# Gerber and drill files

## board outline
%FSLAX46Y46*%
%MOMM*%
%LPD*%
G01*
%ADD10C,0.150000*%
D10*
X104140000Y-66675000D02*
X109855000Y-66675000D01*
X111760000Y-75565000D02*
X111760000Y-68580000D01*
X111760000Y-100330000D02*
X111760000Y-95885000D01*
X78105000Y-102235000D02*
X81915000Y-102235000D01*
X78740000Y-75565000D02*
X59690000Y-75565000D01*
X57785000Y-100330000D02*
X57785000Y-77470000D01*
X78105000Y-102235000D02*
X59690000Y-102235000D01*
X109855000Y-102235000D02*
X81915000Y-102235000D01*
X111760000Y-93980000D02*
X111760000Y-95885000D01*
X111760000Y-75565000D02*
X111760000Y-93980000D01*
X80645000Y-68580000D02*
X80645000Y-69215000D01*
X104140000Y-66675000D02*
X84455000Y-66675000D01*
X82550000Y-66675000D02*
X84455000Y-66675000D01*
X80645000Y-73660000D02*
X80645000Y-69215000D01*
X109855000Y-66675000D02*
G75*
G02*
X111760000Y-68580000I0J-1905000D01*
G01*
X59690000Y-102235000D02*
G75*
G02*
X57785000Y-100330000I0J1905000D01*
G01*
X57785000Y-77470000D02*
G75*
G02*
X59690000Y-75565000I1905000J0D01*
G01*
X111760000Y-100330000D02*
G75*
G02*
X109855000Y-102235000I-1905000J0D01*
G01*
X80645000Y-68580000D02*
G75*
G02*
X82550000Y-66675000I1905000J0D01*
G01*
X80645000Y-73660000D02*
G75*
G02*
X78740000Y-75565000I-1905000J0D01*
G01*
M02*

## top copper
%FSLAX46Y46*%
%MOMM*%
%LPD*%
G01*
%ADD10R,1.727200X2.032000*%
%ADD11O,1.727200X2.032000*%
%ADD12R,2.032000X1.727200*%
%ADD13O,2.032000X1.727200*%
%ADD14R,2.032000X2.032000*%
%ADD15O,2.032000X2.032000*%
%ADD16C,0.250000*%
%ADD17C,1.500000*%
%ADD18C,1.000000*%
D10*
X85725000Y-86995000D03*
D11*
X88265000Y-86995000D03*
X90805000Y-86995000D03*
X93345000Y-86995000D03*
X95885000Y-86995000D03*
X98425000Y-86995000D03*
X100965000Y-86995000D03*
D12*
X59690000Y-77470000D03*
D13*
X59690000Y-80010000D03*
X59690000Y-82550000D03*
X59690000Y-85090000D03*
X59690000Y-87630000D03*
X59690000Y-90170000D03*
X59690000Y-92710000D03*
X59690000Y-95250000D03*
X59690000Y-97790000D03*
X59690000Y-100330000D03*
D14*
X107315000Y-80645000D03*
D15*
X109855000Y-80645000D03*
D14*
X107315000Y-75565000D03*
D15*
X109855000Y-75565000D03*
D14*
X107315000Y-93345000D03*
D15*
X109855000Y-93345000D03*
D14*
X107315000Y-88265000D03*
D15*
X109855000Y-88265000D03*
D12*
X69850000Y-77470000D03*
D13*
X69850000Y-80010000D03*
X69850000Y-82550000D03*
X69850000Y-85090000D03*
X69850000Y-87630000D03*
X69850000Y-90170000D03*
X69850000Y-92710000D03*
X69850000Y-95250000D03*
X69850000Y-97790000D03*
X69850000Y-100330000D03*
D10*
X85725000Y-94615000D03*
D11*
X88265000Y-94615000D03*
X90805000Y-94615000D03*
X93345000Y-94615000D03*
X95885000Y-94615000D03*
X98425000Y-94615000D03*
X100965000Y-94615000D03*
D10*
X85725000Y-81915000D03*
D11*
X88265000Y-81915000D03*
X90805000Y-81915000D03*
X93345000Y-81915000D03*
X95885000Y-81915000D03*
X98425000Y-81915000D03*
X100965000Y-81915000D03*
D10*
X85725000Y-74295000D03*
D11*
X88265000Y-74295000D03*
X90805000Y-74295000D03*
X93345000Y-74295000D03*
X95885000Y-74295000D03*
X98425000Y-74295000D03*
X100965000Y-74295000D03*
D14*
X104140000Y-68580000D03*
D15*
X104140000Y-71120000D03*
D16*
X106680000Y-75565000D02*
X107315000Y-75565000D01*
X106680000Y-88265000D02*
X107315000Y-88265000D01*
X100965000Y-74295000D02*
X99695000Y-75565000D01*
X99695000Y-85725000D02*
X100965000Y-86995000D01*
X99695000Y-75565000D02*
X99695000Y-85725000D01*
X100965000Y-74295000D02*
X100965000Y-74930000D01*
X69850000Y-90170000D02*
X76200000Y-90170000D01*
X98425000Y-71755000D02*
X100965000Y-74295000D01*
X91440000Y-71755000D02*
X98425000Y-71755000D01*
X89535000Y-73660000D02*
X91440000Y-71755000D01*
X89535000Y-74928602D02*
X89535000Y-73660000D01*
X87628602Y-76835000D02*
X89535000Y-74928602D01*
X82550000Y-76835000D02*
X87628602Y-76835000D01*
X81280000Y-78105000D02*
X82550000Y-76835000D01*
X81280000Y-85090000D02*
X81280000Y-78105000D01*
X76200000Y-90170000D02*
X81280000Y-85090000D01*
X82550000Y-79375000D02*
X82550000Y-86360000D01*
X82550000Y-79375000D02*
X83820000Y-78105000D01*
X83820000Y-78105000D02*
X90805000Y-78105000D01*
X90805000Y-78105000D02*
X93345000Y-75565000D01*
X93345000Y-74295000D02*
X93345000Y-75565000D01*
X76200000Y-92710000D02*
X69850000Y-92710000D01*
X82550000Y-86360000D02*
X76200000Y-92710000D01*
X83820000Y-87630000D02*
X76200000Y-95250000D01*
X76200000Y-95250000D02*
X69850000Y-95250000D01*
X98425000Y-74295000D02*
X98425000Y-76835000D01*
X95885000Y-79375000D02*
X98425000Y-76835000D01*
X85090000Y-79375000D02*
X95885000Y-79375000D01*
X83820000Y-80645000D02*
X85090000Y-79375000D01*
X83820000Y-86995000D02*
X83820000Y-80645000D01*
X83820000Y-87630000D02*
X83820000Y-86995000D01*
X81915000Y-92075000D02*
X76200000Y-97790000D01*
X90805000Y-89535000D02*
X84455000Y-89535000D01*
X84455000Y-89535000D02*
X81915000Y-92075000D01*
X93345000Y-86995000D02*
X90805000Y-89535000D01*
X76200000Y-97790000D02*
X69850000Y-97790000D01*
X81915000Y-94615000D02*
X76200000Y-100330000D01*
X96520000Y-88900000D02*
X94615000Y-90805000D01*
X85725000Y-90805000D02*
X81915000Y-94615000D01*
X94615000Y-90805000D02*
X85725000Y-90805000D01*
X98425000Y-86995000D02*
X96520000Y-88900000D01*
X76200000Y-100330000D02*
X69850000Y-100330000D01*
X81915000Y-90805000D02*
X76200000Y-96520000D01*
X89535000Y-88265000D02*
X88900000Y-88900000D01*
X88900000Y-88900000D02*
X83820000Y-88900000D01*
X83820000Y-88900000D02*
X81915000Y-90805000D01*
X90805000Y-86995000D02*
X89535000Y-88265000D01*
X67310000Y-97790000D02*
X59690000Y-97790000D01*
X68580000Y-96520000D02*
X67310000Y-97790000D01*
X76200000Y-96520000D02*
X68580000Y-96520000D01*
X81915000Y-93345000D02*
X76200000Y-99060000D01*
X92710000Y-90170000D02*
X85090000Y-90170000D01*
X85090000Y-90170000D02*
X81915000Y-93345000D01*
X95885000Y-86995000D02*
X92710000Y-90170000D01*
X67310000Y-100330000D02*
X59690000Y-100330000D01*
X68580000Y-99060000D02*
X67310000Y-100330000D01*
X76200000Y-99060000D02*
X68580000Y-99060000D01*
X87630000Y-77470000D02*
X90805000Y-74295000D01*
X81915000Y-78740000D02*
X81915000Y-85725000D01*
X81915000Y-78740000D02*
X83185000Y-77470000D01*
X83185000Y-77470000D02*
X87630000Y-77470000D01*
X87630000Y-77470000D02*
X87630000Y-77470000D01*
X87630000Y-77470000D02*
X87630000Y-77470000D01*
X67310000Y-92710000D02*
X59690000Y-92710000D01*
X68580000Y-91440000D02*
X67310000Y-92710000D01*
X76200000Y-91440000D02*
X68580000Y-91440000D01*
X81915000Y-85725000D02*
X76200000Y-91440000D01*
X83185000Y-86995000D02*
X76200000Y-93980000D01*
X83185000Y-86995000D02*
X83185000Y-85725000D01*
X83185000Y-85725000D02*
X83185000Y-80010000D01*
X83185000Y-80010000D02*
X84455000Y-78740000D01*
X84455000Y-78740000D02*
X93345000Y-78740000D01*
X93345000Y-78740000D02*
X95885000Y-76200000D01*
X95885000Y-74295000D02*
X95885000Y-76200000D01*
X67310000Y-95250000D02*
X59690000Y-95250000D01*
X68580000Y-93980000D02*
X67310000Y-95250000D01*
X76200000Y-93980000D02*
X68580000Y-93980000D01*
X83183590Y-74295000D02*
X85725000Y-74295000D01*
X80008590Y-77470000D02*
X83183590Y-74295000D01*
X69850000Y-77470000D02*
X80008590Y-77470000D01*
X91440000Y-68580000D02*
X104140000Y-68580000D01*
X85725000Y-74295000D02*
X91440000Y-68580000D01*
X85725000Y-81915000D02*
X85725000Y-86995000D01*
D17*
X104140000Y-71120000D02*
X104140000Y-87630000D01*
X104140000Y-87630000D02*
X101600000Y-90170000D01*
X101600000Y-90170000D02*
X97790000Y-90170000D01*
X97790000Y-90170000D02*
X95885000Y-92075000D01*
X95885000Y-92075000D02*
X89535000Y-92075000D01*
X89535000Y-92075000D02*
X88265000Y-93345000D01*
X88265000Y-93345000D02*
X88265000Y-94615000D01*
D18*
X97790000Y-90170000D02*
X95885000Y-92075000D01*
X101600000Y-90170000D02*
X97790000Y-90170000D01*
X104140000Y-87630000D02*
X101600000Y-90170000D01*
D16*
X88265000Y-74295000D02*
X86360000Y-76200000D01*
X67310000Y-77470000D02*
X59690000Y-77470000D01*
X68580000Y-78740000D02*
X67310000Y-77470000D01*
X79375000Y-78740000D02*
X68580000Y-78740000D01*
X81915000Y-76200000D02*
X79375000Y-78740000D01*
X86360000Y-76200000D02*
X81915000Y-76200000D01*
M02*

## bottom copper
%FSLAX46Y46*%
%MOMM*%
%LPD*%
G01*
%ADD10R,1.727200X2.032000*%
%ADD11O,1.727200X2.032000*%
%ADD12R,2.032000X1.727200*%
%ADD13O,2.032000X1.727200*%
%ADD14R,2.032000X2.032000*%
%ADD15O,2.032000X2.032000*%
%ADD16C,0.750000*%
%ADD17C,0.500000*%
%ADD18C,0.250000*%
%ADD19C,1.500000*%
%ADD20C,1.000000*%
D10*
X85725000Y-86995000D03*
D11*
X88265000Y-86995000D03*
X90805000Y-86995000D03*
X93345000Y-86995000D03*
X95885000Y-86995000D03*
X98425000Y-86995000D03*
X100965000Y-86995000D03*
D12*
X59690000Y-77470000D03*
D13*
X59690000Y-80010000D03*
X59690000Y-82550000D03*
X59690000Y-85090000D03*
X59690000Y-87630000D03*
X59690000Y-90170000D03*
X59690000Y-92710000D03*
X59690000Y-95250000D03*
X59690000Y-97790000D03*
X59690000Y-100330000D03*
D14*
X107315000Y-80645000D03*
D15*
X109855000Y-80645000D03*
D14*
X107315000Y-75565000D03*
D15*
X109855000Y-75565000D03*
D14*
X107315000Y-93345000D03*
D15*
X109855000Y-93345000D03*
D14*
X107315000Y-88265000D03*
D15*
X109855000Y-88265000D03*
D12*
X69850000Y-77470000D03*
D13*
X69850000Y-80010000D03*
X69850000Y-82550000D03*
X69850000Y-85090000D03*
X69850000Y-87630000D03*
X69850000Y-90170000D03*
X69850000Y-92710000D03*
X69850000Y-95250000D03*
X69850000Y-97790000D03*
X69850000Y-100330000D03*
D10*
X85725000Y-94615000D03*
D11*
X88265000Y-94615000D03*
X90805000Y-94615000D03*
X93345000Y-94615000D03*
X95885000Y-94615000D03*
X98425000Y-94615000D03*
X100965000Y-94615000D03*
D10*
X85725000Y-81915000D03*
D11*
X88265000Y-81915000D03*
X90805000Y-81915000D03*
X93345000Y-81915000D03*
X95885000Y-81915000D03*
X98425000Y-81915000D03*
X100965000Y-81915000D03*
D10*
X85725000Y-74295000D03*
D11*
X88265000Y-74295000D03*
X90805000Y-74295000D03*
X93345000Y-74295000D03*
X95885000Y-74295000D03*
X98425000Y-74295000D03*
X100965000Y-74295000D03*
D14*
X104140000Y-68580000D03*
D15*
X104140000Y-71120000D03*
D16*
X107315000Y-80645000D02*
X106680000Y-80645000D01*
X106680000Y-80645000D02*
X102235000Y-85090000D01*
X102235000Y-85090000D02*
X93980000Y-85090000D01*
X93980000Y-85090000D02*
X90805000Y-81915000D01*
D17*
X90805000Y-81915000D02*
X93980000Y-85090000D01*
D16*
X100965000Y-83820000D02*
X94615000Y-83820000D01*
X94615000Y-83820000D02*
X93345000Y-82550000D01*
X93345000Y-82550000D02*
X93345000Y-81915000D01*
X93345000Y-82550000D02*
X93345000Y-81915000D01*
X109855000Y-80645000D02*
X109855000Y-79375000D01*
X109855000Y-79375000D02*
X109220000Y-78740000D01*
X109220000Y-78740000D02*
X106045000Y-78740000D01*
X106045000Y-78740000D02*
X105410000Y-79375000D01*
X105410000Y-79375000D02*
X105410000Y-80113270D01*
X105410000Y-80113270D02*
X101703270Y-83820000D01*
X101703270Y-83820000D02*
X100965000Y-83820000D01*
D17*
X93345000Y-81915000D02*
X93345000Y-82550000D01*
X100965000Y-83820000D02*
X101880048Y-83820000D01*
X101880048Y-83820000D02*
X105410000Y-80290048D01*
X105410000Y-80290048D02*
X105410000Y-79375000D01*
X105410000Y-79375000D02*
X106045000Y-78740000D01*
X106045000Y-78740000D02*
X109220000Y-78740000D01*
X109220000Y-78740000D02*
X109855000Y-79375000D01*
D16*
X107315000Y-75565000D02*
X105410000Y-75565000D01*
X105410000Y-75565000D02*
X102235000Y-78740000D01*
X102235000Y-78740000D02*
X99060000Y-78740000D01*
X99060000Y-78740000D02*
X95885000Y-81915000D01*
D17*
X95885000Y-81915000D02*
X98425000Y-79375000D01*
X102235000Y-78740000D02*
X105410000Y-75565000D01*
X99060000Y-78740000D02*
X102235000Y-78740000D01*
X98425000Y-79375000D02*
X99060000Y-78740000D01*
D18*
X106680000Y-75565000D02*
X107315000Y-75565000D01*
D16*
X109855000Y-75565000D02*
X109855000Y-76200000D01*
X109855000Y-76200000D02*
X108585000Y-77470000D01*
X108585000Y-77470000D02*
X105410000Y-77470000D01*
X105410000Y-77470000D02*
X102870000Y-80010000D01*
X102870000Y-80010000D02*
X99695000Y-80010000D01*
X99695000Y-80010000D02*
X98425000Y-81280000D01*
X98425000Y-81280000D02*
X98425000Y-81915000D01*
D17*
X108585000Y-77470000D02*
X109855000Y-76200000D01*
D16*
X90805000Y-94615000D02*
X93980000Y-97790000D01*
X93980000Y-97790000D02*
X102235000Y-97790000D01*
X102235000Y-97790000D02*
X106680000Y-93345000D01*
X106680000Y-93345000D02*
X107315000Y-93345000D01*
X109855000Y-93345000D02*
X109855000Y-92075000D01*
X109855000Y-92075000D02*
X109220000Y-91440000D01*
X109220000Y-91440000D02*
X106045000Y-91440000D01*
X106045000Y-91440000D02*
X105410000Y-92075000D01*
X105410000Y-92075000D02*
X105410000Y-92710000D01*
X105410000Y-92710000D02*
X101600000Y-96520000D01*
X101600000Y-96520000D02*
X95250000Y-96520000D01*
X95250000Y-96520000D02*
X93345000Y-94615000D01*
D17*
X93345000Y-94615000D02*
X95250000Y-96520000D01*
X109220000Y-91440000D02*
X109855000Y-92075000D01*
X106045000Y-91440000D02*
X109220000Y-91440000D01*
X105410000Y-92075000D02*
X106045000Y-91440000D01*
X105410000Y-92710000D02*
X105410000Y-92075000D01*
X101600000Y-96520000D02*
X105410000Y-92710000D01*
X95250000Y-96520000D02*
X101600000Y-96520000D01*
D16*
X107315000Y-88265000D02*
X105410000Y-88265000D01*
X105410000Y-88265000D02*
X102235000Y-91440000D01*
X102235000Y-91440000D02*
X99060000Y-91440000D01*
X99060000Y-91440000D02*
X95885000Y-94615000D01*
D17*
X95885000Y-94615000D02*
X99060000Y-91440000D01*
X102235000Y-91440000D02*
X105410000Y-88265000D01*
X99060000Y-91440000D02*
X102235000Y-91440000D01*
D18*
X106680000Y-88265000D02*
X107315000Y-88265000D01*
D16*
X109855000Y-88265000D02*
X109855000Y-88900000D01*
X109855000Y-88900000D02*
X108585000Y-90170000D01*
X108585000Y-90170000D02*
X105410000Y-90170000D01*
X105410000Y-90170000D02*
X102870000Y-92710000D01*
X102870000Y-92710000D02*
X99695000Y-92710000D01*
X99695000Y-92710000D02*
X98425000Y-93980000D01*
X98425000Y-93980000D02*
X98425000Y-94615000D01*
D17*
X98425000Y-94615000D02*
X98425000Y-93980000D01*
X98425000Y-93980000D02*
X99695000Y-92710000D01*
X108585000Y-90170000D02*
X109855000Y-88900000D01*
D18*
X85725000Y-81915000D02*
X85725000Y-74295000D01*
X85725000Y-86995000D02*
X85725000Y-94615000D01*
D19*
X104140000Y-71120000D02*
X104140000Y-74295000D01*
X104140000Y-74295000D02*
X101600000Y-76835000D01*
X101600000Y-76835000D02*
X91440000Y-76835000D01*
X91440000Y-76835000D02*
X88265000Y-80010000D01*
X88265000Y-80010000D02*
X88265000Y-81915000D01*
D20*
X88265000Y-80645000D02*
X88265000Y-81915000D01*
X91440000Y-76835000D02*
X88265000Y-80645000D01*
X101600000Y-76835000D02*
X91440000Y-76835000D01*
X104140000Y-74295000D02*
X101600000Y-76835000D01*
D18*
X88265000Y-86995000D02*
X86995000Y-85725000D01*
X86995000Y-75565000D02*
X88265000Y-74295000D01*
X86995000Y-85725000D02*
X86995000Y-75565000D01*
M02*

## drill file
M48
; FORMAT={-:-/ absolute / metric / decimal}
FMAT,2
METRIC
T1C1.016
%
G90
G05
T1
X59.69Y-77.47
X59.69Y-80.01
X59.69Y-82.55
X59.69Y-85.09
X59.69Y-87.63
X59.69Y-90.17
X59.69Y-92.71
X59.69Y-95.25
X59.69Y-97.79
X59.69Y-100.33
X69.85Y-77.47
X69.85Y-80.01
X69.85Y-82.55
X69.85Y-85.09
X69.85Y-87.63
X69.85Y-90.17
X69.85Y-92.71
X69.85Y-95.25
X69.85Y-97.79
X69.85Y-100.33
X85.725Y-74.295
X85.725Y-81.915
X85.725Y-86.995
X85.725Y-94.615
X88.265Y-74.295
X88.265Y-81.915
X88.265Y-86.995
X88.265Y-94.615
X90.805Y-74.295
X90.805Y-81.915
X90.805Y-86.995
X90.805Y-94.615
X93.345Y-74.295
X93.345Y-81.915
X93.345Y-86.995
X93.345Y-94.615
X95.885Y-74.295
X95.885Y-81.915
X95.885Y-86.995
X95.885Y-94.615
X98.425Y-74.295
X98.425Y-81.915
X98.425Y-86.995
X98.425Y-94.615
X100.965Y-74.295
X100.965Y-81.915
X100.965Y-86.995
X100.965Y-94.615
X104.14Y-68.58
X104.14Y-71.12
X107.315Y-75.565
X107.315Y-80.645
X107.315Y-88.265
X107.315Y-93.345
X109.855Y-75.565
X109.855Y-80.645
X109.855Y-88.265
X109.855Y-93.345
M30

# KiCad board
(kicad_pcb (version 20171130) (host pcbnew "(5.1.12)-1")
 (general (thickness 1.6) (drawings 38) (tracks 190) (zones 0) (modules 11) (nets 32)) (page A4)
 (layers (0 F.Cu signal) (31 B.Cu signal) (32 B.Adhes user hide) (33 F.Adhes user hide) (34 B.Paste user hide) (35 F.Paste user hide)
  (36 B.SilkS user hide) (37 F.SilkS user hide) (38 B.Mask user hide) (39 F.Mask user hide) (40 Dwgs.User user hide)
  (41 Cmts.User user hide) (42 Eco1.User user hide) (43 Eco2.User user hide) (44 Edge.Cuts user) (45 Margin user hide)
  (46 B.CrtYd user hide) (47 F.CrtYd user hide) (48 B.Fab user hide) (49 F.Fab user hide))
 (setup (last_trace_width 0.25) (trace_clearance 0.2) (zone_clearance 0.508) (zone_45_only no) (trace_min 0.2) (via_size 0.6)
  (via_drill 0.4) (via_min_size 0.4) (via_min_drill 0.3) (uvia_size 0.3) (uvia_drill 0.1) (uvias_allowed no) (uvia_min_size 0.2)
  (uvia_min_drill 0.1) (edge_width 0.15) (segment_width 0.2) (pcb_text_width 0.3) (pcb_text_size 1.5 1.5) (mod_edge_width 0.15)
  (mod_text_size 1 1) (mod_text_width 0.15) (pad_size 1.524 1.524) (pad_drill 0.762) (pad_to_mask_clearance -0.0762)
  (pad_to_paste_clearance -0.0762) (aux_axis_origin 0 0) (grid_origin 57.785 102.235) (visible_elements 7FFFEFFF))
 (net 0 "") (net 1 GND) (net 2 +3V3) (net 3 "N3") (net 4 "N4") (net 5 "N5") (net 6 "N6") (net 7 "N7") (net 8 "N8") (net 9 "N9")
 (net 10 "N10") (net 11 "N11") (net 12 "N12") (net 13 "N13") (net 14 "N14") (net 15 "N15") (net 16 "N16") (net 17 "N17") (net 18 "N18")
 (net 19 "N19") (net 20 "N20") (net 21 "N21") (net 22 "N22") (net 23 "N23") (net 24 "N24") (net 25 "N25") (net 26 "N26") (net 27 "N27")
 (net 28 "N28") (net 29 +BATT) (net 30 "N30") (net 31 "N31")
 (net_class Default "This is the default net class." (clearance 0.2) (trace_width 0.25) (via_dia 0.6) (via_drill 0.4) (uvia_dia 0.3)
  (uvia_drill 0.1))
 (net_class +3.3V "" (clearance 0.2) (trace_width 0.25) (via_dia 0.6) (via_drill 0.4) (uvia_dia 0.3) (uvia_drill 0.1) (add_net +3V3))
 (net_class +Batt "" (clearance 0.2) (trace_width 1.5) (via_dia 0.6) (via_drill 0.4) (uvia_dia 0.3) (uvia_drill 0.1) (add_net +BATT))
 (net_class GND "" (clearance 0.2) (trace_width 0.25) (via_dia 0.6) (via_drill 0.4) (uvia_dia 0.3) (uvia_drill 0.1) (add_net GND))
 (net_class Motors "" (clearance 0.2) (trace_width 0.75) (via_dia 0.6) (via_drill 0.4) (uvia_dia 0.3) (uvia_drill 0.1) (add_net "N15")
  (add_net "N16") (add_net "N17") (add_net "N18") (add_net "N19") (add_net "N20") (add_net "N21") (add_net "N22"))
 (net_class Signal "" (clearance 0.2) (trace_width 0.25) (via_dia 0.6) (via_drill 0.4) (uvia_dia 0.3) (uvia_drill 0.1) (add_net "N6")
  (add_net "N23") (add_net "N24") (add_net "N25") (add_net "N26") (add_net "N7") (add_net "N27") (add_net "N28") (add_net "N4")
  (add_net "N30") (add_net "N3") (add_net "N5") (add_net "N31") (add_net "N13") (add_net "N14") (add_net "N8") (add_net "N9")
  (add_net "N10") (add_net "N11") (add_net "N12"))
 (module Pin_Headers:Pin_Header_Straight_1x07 (layer F.Cu) (at 85.725 86.995 90)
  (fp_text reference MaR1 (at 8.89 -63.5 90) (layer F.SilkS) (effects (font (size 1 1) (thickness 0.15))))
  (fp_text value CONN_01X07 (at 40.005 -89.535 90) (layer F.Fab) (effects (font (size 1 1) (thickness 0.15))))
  (pad 1 thru_hole rect (at 0 0 90) (size 2.032 1.7272) (drill 1.016) (layers *.Cu *.Mask F.SilkS) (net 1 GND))
  (pad 2 thru_hole oval (at 0 2.54 90) (size 2.032 1.7272) (drill 1.016) (layers *.Cu *.Mask F.SilkS) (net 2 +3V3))
  (pad 3 thru_hole oval (at 0 5.08 90) (size 2.032 1.7272) (drill 1.016) (layers *.Cu *.Mask F.SilkS) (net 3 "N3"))
  (pad 4 thru_hole oval (at 0 7.62 90) (size 2.032 1.7272) (drill 1.016) (layers *.Cu *.Mask F.SilkS) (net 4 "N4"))
  (pad 5 thru_hole oval (at 0 10.16 90) (size 2.032 1.7272) (drill 1.016) (layers *.Cu *.Mask F.SilkS) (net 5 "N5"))
  (pad 6 thru_hole oval (at 0 12.7 90) (size 2.032 1.7272) (drill 1.016) (layers *.Cu *.Mask F.SilkS) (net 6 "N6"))
  (pad 7 thru_hole oval (at 0 15.24 90) (size 2.032 1.7272) (drill 1.016) (layers *.Cu *.Mask F.SilkS) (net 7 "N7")))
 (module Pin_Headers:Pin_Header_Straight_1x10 (layer F.Cu) (at 59.69 77.47)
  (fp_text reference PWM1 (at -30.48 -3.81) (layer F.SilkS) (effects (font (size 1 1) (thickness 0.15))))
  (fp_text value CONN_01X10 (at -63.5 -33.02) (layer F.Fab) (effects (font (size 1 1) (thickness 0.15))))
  (pad 1 thru_hole rect (at 0 0) (size 2.032 1.7272) (drill 1.016) (layers *.Cu *.Mask F.SilkS) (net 2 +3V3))
  (pad 2 thru_hole oval (at 0 2.54) (size 2.032 1.7272) (drill 1.016) (layers *.Cu *.Mask F.SilkS) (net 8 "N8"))
  (pad 3 thru_hole oval (at 0 5.08) (size 2.032 1.7272) (drill 1.016) (layers *.Cu *.Mask F.SilkS) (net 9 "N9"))
  (pad 4 thru_hole oval (at 0 7.62) (size 2.032 1.7272) (drill 1.016) (layers *.Cu *.Mask F.SilkS) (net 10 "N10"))
  (pad 5 thru_hole oval (at 0 10.16) (size 2.032 1.7272) (drill 1.016) (layers *.Cu *.Mask F.SilkS) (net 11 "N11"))
  (pad 6 thru_hole oval (at 0 12.7) (size 2.032 1.7272) (drill 1.016) (layers *.Cu *.Mask F.SilkS) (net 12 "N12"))
  (pad 7 thru_hole oval (at 0 15.24) (size 2.032 1.7272) (drill 1.016) (layers *.Cu *.Mask F.SilkS) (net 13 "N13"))
  (pad 8 thru_hole oval (at 0 17.78) (size 2.032 1.7272) (drill 1.016) (layers *.Cu *.Mask F.SilkS) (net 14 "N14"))
  (pad 9 thru_hole oval (at 0 20.32) (size 2.032 1.7272) (drill 1.016) (layers *.Cu *.Mask F.SilkS) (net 3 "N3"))
  (pad 10 thru_hole oval (at 0 22.86) (size 2.032 1.7272) (drill 1.016) (layers *.Cu *.Mask F.SilkS) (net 5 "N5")))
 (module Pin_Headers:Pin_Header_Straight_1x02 (layer F.Cu) (at 107.315 80.645 90)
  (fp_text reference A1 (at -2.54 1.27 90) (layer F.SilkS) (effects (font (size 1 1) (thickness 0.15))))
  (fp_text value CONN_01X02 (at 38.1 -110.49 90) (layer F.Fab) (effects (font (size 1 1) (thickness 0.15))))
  (pad 1 thru_hole rect (at 0 0 90) (size 2.032 2.032) (drill 1.016) (layers *.Cu *.Mask F.SilkS) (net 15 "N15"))
  (pad 2 thru_hole oval (at 0 2.54 90) (size 2.032 2.032) (drill 1.016) (layers *.Cu *.Mask F.SilkS) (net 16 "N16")))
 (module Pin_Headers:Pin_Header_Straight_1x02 (layer F.Cu) (at 107.315 75.565 90)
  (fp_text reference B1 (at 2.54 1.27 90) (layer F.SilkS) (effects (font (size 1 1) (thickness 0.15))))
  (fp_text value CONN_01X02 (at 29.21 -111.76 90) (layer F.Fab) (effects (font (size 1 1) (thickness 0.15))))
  (pad 1 thru_hole rect (at 0 0 90) (size 2.032 2.032) (drill 1.016) (layers *.Cu *.Mask F.SilkS) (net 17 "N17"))
  (pad 2 thru_hole oval (at 0 2.54 90) (size 2.032 2.032) (drill 1.016) (layers *.Cu *.Mask F.SilkS) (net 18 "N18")))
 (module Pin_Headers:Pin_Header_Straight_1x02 (layer F.Cu) (at 107.315 93.345 90)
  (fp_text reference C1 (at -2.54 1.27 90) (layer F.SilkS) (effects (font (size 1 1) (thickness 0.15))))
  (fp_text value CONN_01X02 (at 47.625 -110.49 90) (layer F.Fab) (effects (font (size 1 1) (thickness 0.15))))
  (pad 1 thru_hole rect (at 0 0 90) (size 2.032 2.032) (drill 1.016) (layers *.Cu *.Mask F.SilkS) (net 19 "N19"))
  (pad 2 thru_hole oval (at 0 2.54 90) (size 2.032 2.032) (drill 1.016) (layers *.Cu *.Mask F.SilkS) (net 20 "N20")))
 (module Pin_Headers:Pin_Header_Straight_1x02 (layer F.Cu) (at 107.315 88.265 90)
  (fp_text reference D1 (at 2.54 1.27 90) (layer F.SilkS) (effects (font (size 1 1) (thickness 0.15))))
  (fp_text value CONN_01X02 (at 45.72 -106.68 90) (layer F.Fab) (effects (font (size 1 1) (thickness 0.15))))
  (pad 1 thru_hole rect (at 0 0 90) (size 2.032 2.032) (drill 1.016) (layers *.Cu *.Mask F.SilkS) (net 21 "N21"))
  (pad 2 thru_hole oval (at 0 2.54 90) (size 2.032 2.032) (drill 1.016) (layers *.Cu *.Mask F.SilkS) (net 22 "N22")))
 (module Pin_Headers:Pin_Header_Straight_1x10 (layer F.Cu) (at 69.85 77.47)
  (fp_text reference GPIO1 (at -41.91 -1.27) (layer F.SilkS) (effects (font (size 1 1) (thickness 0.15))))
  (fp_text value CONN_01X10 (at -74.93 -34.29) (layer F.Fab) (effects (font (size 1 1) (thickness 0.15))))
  (pad 1 thru_hole rect (at 0 0) (size 2.032 1.7272) (drill 1.016) (layers *.Cu *.Mask F.SilkS) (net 1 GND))
  (pad 2 thru_hole oval (at 0 2.54) (size 2.032 1.7272) (drill 1.016) (layers *.Cu *.Mask F.SilkS) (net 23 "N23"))
  (pad 3 thru_hole oval (at 0 5.08) (size 2.032 1.7272) (drill 1.016) (layers *.Cu *.Mask F.SilkS) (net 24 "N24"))
  (pad 4 thru_hole oval (at 0 7.62) (size 2.032 1.7272) (drill 1.016) (layers *.Cu *.Mask F.SilkS) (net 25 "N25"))
  (pad 5 thru_hole oval (at 0 10.16) (size 2.032 1.7272) (drill 1.016) (layers *.Cu *.Mask F.SilkS) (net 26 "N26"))
  (pad 6 thru_hole oval (at 0 12.7) (size 2.032 1.7272) (drill 1.016) (layers *.Cu *.Mask F.SilkS) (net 7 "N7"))
  (pad 7 thru_hole oval (at 0 15.24) (size 2.032 1.7272) (drill 1.016) (layers *.Cu *.Mask F.SilkS) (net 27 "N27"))
  (pad 8 thru_hole oval (at 0 17.78) (size 2.032 1.7272) (drill 1.016) (layers *.Cu *.Mask F.SilkS) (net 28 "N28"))
  (pad 9 thru_hole oval (at 0 20.32) (size 2.032 1.7272) (drill 1.016) (layers *.Cu *.Mask F.SilkS) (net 4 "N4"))
  (pad 10 thru_hole oval (at 0 22.86) (size 2.032 1.7272) (drill 1.016) (layers *.Cu *.Mask F.SilkS) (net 6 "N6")))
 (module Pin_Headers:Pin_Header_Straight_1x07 (layer F.Cu) (at 85.725 94.615 90)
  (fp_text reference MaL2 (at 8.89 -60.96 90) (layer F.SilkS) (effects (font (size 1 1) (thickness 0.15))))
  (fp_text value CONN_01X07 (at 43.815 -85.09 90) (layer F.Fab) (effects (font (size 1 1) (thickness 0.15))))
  (pad 1 thru_hole rect (at 0 0 90) (size 2.032 1.7272) (drill 1.016) (layers *.Cu *.Mask F.SilkS) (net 1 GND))
  (pad 2 thru_hole oval (at 0 2.54 90) (size 2.032 1.7272) (drill 1.016) (layers *.Cu *.Mask F.SilkS) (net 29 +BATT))
  (pad 3 thru_hole oval (at 0 5.08 90) (size 2.032 1.7272) (drill 1.016) (layers *.Cu *.Mask F.SilkS) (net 19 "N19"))
  (pad 4 thru_hole oval (at 0 7.62 90) (size 2.032 1.7272) (drill 1.016) (layers *.Cu *.Mask F.SilkS) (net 20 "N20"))
  (pad 5 thru_hole oval (at 0 10.16 90) (size 2.032 1.7272) (drill 1.016) (layers *.Cu *.Mask F.SilkS) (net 21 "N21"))
  (pad 6 thru_hole oval (at 0 12.7 90) (size 2.032 1.7272) (drill 1.016) (layers *.Cu *.Mask F.SilkS) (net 22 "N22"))
  (pad 7 thru_hole oval (at 0 15.24 90) (size 2.032 1.7272) (drill 1.016) (layers *.Cu *.Mask F.SilkS) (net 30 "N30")))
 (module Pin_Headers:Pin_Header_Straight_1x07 (layer F.Cu) (at 85.725 81.915 90)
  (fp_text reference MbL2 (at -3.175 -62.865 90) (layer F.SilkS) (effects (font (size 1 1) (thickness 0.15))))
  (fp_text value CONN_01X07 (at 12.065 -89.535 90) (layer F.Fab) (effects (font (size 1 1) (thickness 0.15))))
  (pad 1 thru_hole rect (at 0 0 90) (size 2.032 1.7272) (drill 1.016) (layers *.Cu *.Mask F.SilkS) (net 1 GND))
  (pad 2 thru_hole oval (at 0 2.54 90) (size 2.032 1.7272) (drill 1.016) (layers *.Cu *.Mask F.SilkS) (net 29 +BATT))
  (pad 3 thru_hole oval (at 0 5.08 90) (size 2.032 1.7272) (drill 1.016) (layers *.Cu *.Mask F.SilkS) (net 15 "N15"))
  (pad 4 thru_hole oval (at 0 7.62 90) (size 2.032 1.7272) (drill 1.016) (layers *.Cu *.Mask F.SilkS) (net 16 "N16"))
  (pad 5 thru_hole oval (at 0 10.16 90) (size 2.032 1.7272) (drill 1.016) (layers *.Cu *.Mask F.SilkS) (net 17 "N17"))
  (pad 6 thru_hole oval (at 0 12.7 90) (size 2.032 1.7272) (drill 1.016) (layers *.Cu *.Mask F.SilkS) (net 18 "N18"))
  (pad 7 thru_hole oval (at 0 15.24 90) (size 2.032 1.7272) (drill 1.016) (layers *.Cu *.Mask F.SilkS) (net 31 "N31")))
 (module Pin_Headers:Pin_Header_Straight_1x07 (layer F.Cu) (at 85.725 74.295 90)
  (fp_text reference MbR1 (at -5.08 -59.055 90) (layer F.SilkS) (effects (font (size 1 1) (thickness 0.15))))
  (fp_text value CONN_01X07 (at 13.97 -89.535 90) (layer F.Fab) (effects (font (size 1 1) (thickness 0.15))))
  (pad 1 thru_hole rect (at 0 0 90) (size 2.032 1.7272) (drill 1.016) (layers *.Cu *.Mask F.SilkS) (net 1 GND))
  (pad 2 thru_hole oval (at 0 2.54 90) (size 2.032 1.7272) (drill 1.016) (layers *.Cu *.Mask F.SilkS) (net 2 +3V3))
  (pad 3 thru_hole oval (at 0 5.08 90) (size 2.032 1.7272) (drill 1.016) (layers *.Cu *.Mask F.SilkS) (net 13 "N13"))
  (pad 4 thru_hole oval (at 0 7.62 90) (size 2.032 1.7272) (drill 1.016) (layers *.Cu *.Mask F.SilkS) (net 27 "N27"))
  (pad 5 thru_hole oval (at 0 10.16 90) (size 2.032 1.7272) (drill 1.016) (layers *.Cu *.Mask F.SilkS) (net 14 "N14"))
  (pad 6 thru_hole oval (at 0 12.7 90) (size 2.032 1.7272) (drill 1.016) (layers *.Cu *.Mask F.SilkS) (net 28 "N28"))
  (pad 7 thru_hole oval (at 0 15.24 90) (size 2.032 1.7272) (drill 1.016) (layers *.Cu *.Mask F.SilkS) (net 7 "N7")))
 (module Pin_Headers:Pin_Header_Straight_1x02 (layer F.Cu) (at 104.14 68.58)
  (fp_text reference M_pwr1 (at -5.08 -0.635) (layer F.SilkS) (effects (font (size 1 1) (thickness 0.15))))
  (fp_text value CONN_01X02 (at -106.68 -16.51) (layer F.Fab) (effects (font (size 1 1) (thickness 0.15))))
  (pad 1 thru_hole rect (at 0 0) (size 2.032 2.032) (drill 1.016) (layers *.Cu *.Mask F.SilkS) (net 1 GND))
  (pad 2 thru_hole oval (at 0 2.54) (size 2.032 2.032) (drill 1.016) (layers *.Cu *.Mask F.SilkS) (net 29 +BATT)))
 (gr_line (start 104.14 66.675) (end 109.855 66.675) (angle 90) (layer Edge.Cuts) (width 0.15))
 (gr_line (start 111.76 75.565) (end 111.76 68.58) (angle 90) (layer Edge.Cuts) (width 0.15))
 (gr_line (start 111.76 100.33) (end 111.76 95.885) (angle 90) (layer Edge.Cuts) (width 0.15))
 (gr_line (start 78.105 102.235) (end 81.915 102.235) (angle 90) (layer Edge.Cuts) (width 0.15))
 (gr_line (start 78.74 75.565) (end 59.69 75.565) (angle 90) (layer Edge.Cuts) (width 0.15))
 (gr_line (start 57.785 100.33) (end 57.785 77.47) (angle 90) (layer Edge.Cuts) (width 0.15))
 (gr_line (start 78.105 102.235) (end 59.69 102.235) (angle 90) (layer Edge.Cuts) (width 0.15))
 (gr_line (start 109.855 102.235) (end 81.915 102.235) (angle 90) (layer Edge.Cuts) (width 0.15))
 (gr_line (start 111.76 93.98) (end 111.76 95.885) (angle 90) (layer Edge.Cuts) (width 0.15))
 (gr_line (start 111.76 75.565) (end 111.76 93.98) (angle 90) (layer Edge.Cuts) (width 0.15))
 (gr_line (start 80.645 68.58) (end 80.645 69.215) (angle 90) (layer Edge.Cuts) (width 0.15))
 (gr_line (start 104.14 66.675) (end 84.455 66.675) (angle 90) (layer Edge.Cuts) (width 0.15))
 (gr_line (start 82.55 66.675) (end 84.455 66.675) (angle 90) (layer Edge.Cuts) (width 0.15))
 (gr_line (start 80.645 73.66) (end 80.645 69.215) (angle 90) (layer Edge.Cuts) (width 0.15))
 (gr_arc (start 109.855 68.58) (end 109.855 66.675) (angle 90) (layer Edge.Cuts) (width 0.15))
 (gr_arc (start 59.69 100.33) (end 59.69 102.235) (angle 90) (layer Edge.Cuts) (width 0.15))
 (gr_arc (start 59.69 77.47) (end 57.785 77.47) (angle 90) (layer Edge.Cuts) (width 0.15))
 (gr_arc (start 109.855 100.33) (end 111.76 100.33) (angle 90) (layer Edge.Cuts) (width 0.15))
 (gr_arc (start 82.55 68.58) (end 80.645 68.58) (angle 90) (layer Edge.Cuts) (width 0.15))
 (gr_arc (start 78.74 73.66) (end 80.645 73.66) (angle 90) (layer Edge.Cuts) (width 0.15))
 (segment (start 107.315 80.645) (end 106.68 80.645) (width 0.75) (layer B.Cu) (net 15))
 (segment (start 106.68 80.645) (end 102.235 85.09) (width 0.75) (layer B.Cu) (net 15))
 (segment (start 102.235 85.09) (end 93.98 85.09) (width 0.75) (layer B.Cu) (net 15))
 (segment (start 93.98 85.09) (end 90.805 81.915) (width 0.75) (layer B.Cu) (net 15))
 (segment (start 90.805 81.915) (end 93.98 85.09) (width 0.5) (layer B.Cu) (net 15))
 (segment (start 100.965 83.82) (end 94.615 83.82) (width 0.75) (layer B.Cu) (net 16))
 (segment (start 94.615 83.82) (end 93.345 82.55) (width 0.75) (layer B.Cu) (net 16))
 (segment (start 93.345 82.55) (end 93.345 81.915) (width 0.75) (layer B.Cu) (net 16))
 (segment (start 93.345 82.55) (end 93.345 81.915) (width 0.75) (layer B.Cu) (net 16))
 (segment (start 109.855 80.645) (end 109.855 79.375) (width 0.75) (layer B.Cu) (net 16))
 (segment (start 109.855 79.375) (end 109.22 78.74) (width 0.75) (layer B.Cu) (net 16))
 (segment (start 109.22 78.74) (end 106.045 78.74) (width 0.75) (layer B.Cu) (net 16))
 (segment (start 106.045 78.74) (end 105.41 79.375) (width 0.75) (layer B.Cu) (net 16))
 (segment (start 105.41 79.375) (end 105.41 80.11327) (width 0.75) (layer B.Cu) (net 16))
 (segment (start 105.41 80.11327) (end 101.70327 83.82) (width 0.75) (layer B.Cu) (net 16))
 (segment (start 101.70327 83.82) (end 100.965 83.82) (width 0.75) (layer B.Cu) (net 16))
 (segment (start 93.345 81.915) (end 93.345 82.55) (width 0.5) (layer B.Cu) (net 16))
 (segment (start 100.965 83.82) (end 101.880048 83.82) (width 0.5) (layer B.Cu) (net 16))
 (segment (start 101.880048 83.82) (end 105.41 80.290048) (width 0.5) (layer B.Cu) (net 16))
 (segment (start 105.41 80.290048) (end 105.41 79.375) (width 0.5) (layer B.Cu) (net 16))
 (segment (start 105.41 79.375) (end 106.045 78.74) (width 0.5) (layer B.Cu) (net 16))
 (segment (start 106.045 78.74) (end 109.22 78.74) (width 0.5) (layer B.Cu) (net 16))
 (segment (start 109.22 78.74) (end 109.855 79.375) (width 0.5) (layer B.Cu) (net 16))
 (segment (start 107.315 75.565) (end 105.41 75.565) (width 0.75) (layer B.Cu) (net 17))
 (segment (start 105.41 75.565) (end 102.235 78.74) (width 0.75) (layer B.Cu) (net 17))
 (segment (start 102.235 78.74) (end 99.06 78.74) (width 0.75) (layer B.Cu) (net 17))
 (segment (start 99.06 78.74) (end 95.885 81.915) (width 0.75) (layer B.Cu) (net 17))
 (segment (start 95.885 81.915) (end 98.425 79.375) (width 0.5) (layer B.Cu) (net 17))
 (segment (start 102.235 78.74) (end 105.41 75.565) (width 0.5) (layer B.Cu) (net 17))
 (segment (start 99.06 78.74) (end 102.235 78.74) (width 0.5) (layer B.Cu) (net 17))
 (segment (start 98.425 79.375) (end 99.06 78.74) (width 0.5) (layer B.Cu) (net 17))
 (segment (start 106.68 75.565) (end 107.315 75.565) (width 0.25) (layer B.Cu) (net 17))
 (segment (start 106.68 75.565) (end 107.315 75.565) (width 0.25) (layer F.Cu) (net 17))
 (segment (start 109.855 75.565) (end 109.855 76.2) (width 0.75) (layer B.Cu) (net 18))
 (segment (start 109.855 76.2) (end 108.585 77.47) (width 0.75) (layer B.Cu) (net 18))
 (segment (start 108.585 77.47) (end 105.41 77.47) (width 0.75) (layer B.Cu) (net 18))
 (segment (start 105.41 77.47) (end 102.87 80.01) (width 0.75) (layer B.Cu) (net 18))
 (segment (start 102.87 80.01) (end 99.695 80.01) (width 0.75) (layer B.Cu) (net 18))
 (segment (start 99.695 80.01) (end 98.425 81.28) (width 0.75) (layer B.Cu) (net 18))
 (segment (start 98.425 81.28) (end 98.425 81.915) (width 0.75) (layer B.Cu) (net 18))
 (segment (start 108.585 77.47) (end 109.855 76.2) (width 0.5) (layer B.Cu) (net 18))
 (segment (start 90.805 94.615) (end 93.98 97.79) (width 0.75) (layer B.Cu) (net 19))
 (segment (start 93.98 97.79) (end 102.235 97.79) (width 0.75) (layer B.Cu) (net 19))
 (segment (start 102.235 97.79) (end 106.68 93.345) (width 0.75) (layer B.Cu) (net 19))
 (segment (start 106.68 93.345) (end 107.315 93.345) (width 0.75) (layer B.Cu) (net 19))
 (segment (start 109.855 93.345) (end 109.855 92.075) (width 0.75) (layer B.Cu) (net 20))
 (segment (start 109.855 92.075) (end 109.22 91.44) (width 0.75) (layer B.Cu) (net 20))
 (segment (start 109.22 91.44) (end 106.045 91.44) (width 0.75) (layer B.Cu) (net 20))
 (segment (start 106.045 91.44) (end 105.41 92.075) (width 0.75) (layer B.Cu) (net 20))
 (segment (start 105.41 92.075) (end 105.41 92.71) (width 0.75) (layer B.Cu) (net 20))
 (segment (start 105.41 92.71) (end 101.6 96.52) (width 0.75) (layer B.Cu) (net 20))
 (segment (start 101.6 96.52) (end 95.25 96.52) (width 0.75) (layer B.Cu) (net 20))
 (segment (start 95.25 96.52) (end 93.345 94.615) (width 0.75) (layer B.Cu) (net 20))
 (segment (start 93.345 94.615) (end 95.25 96.52) (width 0.5) (layer B.Cu) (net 20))
 (segment (start 109.22 91.44) (end 109.855 92.075) (width 0.5) (layer B.Cu) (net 20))
 (segment (start 106.045 91.44) (end 109.22 91.44) (width 0.5) (layer B.Cu) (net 20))
 (segment (start 105.41 92.075) (end 106.045 91.44) (width 0.5) (layer B.Cu) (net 20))
 (segment (start 105.41 92.71) (end 105.41 92.075) (width 0.5) (layer B.Cu) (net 20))
 (segment (start 101.6 96.52) (end 105.41 92.71) (width 0.5) (layer B.Cu) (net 20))
 (segment (start 95.25 96.52) (end 101.6 96.52) (width 0.5) (layer B.Cu) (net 20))
 (segment (start 107.315 88.265) (end 105.41 88.265) (width 0.75) (layer B.Cu) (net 21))
 (segment (start 105.41 88.265) (end 102.235 91.44) (width 0.75) (layer B.Cu) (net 21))
 (segment (start 102.235 91.44) (end 99.06 91.44) (width 0.75) (layer B.Cu) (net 21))
 (segment (start 99.06 91.44) (end 95.885 94.615) (width 0.75) (layer B.Cu) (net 21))
 (segment (start 95.885 94.615) (end 99.06 91.44) (width 0.5) (layer B.Cu) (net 21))
 (segment (start 102.235 91.44) (end 105.41 88.265) (width 0.5) (layer B.Cu) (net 21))
 (segment (start 99.06 91.44) (end 102.235 91.44) (width 0.5) (layer B.Cu) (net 21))
 (segment (start 106.68 88.265) (end 107.315 88.265) (width 0.25) (layer B.Cu) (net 21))
 (segment (start 106.68 88.265) (end 107.315 88.265) (width 0.25) (layer F.Cu) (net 21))
 (segment (start 109.855 88.265) (end 109.855 88.9) (width 0.75) (layer B.Cu) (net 22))
 (segment (start 109.855 88.9) (end 108.585 90.17) (width 0.75) (layer B.Cu) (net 22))
 (segment (start 108.585 90.17) (end 105.41 90.17) (width 0.75) (layer B.Cu) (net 22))
 (segment (start 105.41 90.17) (end 102.87 92.71) (width 0.75) (layer B.Cu) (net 22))
 (segment (start 102.87 92.71) (end 99.695 92.71) (width 0.75) (layer B.Cu) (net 22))
 (segment (start 99.695 92.71) (end 98.425 93.98) (width 0.75) (layer B.Cu) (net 22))
 (segment (start 98.425 93.98) (end 98.425 94.615) (width 0.75) (layer B.Cu) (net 22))
 (segment (start 98.425 94.615) (end 98.425 93.98) (width 0.5) (layer B.Cu) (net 22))
 (segment (start 98.425 93.98) (end 99.695 92.71) (width 0.5) (layer B.Cu) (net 22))
 (segment (start 108.585 90.17) (end 109.855 88.9) (width 0.5) (layer B.Cu) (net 22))
 (segment (start 100.965 74.295) (end 99.695 75.565) (width 0.25) (layer F.Cu) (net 7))
 (segment (start 99.695 85.725) (end 100.965 86.995) (width 0.25) (layer F.Cu) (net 7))
 (segment (start 99.695 75.565) (end 99.695 85.725) (width 0.25) (layer F.Cu) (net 7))
 (segment (start 100.965 74.295) (end 100.965 74.93) (width 0.25) (layer F.Cu) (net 7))
 (segment (start 69.85 90.17) (end 76.2 90.17) (width 0.25) (layer F.Cu) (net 7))
 (segment (start 98.425 71.755) (end 100.965 74.295) (width 0.25) (layer F.Cu) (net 7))
 (segment (start 91.44 71.755) (end 98.425 71.755) (width 0.25) (layer F.Cu) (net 7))
 (segment (start 89.535 73.66) (end 91.44 71.755) (width 0.25) (layer F.Cu) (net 7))
 (segment (start 89.535 74.928602) (end 89.535 73.66) (width 0.25) (layer F.Cu) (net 7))
 (segment (start 87.628602 76.835) (end 89.535 74.928602) (width 0.25) (layer F.Cu) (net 7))
 (segment (start 82.55 76.835) (end 87.628602 76.835) (width 0.25) (layer F.Cu) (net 7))
 (segment (start 81.28 78.105) (end 82.55 76.835) (width 0.25) (layer F.Cu) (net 7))
 (segment (start 81.28 85.09) (end 81.28 78.105) (width 0.25) (layer F.Cu) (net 7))
 (segment (start 76.2 90.17) (end 81.28 85.09) (width 0.25) (layer F.Cu) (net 7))
 (segment (start 82.55 79.375) (end 82.55 86.36) (width 0.25) (layer F.Cu) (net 27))
 (segment (start 82.55 79.375) (end 83.82 78.105) (width 0.25) (layer F.Cu) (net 27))
 (segment (start 83.82 78.105) (end 90.805 78.105) (width 0.25) (layer F.Cu) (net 27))
 (segment (start 90.805 78.105) (end 93.345 75.565) (width 0.25) (layer F.Cu) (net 27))
 (segment (start 93.345 74.295) (end 93.345 75.565) (width 0.25) (layer F.Cu) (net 27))
 (segment (start 76.2 92.71) (end 69.85 92.71) (width 0.25) (layer F.Cu) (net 27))
 (segment (start 82.55 86.36) (end 76.2 92.71) (width 0.25) (layer F.Cu) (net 27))
 (segment (start 83.82 87.63) (end 76.2 95.25) (width 0.25) (layer F.Cu) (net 28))
 (segment (start 76.2 95.25) (end 69.85 95.25) (width 0.25) (layer F.Cu) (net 28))
 (segment (start 98.425 74.295) (end 98.425 76.835) (width 0.25) (layer F.Cu) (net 28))
 (segment (start 95.885 79.375) (end 98.425 76.835) (width 0.25) (layer F.Cu) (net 28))
 (segment (start 85.09 79.375) (end 95.885 79.375) (width 0.25) (layer F.Cu) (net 28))
 (segment (start 83.82 80.645) (end 85.09 79.375) (width 0.25) (layer F.Cu) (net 28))
 (segment (start 83.82 86.995) (end 83.82 80.645) (width 0.25) (layer F.Cu) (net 28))
 (segment (start 83.82 87.63) (end 83.82 86.995) (width 0.25) (layer F.Cu) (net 28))
 (segment (start 81.915 92.075) (end 76.2 97.79) (width 0.25) (layer F.Cu) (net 4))
 (segment (start 90.805 89.535) (end 84.455 89.535) (width 0.25) (layer F.Cu) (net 4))
 (segment (start 84.455 89.535) (end 81.915 92.075) (width 0.25) (layer F.Cu) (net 4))
 (segment (start 93.345 86.995) (end 90.805 89.535) (width 0.25) (layer F.Cu) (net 4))
 (segment (start 76.2 97.79) (end 69.85 97.79) (width 0.25) (layer F.Cu) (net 4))
 (segment (start 81.915 94.615) (end 76.2 100.33) (width 0.25) (layer F.Cu) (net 6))
 (segment (start 96.52 88.9) (end 94.615 90.805) (width 0.25) (layer F.Cu) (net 6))
 (segment (start 85.725 90.805) (end 81.915 94.615) (width 0.25) (layer F.Cu) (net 6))
 (segment (start 94.615 90.805) (end 85.725 90.805) (width 0.25) (layer F.Cu) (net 6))
 (segment (start 98.425 86.995) (end 96.52 88.9) (width 0.25) (layer F.Cu) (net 6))
 (segment (start 76.2 100.33) (end 69.85 100.33) (width 0.25) (layer F.Cu) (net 6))
 (segment (start 81.915 90.805) (end 76.2 96.52) (width 0.25) (layer F.Cu) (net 3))
 (segment (start 89.535 88.265) (end 88.9 88.9) (width 0.25) (layer F.Cu) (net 3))
 (segment (start 88.9 88.9) (end 83.82 88.9) (width 0.25) (layer F.Cu) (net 3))
 (segment (start 83.82 88.9) (end 81.915 90.805) (width 0.25) (layer F.Cu) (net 3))
 (segment (start 90.805 86.995) (end 89.535 88.265) (width 0.25) (layer F.Cu) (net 3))
 (segment (start 67.31 97.79) (end 59.69 97.79) (width 0.25) (layer F.Cu) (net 3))
 (segment (start 68.58 96.52) (end 67.31 97.79) (width 0.25) (layer F.Cu) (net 3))
 (segment (start 76.2 96.52) (end 68.58 96.52) (width 0.25) (layer F.Cu) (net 3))
 (segment (start 81.915 93.345) (end 76.2 99.06) (width 0.25) (layer F.Cu) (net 5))
 (segment (start 92.71 90.17) (end 85.09 90.17) (width 0.25) (layer F.Cu) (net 5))
 (segment (start 85.09 90.17) (end 81.915 93.345) (width 0.25) (layer F.Cu) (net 5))
 (segment (start 95.885 86.995) (end 92.71 90.17) (width 0.25) (layer F.Cu) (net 5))
 (segment (start 67.31 100.33) (end 59.69 100.33) (width 0.25) (layer F.Cu) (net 5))
 (segment (start 68.58 99.06) (end 67.31 100.33) (width 0.25) (layer F.Cu) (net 5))
 (segment (start 76.2 99.06) (end 68.58 99.06) (width 0.25) (layer F.Cu) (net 5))
 (segment (start 87.63 77.47) (end 90.805 74.295) (width 0.25) (layer F.Cu) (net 13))
 (segment (start 81.915 78.74) (end 81.915 85.725) (width 0.25) (layer F.Cu) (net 13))
 (segment (start 81.915 78.74) (end 83.185 77.47) (width 0.25) (layer F.Cu) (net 13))
 (segment (start 83.185 77.47) (end 87.63 77.47) (width 0.25) (layer F.Cu) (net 13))
 (segment (start 87.63 77.47) (end 87.63 77.47) (width 0.25) (layer F.Cu) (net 13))
 (segment (start 87.63 77.47) (end 87.63 77.47) (width 0.25) (layer F.Cu) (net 13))
 (segment (start 67.31 92.71) (end 59.69 92.71) (width 0.25) (layer F.Cu) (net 13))
 (segment (start 68.58 91.44) (end 67.31 92.71) (width 0.25) (layer F.Cu) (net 13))
 (segment (start 76.2 91.44) (end 68.58 91.44) (width 0.25) (layer F.Cu) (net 13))
 (segment (start 81.915 85.725) (end 76.2 91.44) (width 0.25) (layer F.Cu) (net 13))
 (segment (start 83.185 86.995) (end 76.2 93.98) (width 0.25) (layer F.Cu) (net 14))
 (segment (start 83.185 86.995) (end 83.185 85.725) (width 0.25) (layer F.Cu) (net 14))
 (segment (start 83.185 85.725) (end 83.185 80.01) (width 0.25) (layer F.Cu) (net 14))
 (segment (start 83.185 80.01) (end 84.455 78.74) (width 0.25) (layer F.Cu) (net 14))
 (segment (start 84.455 78.74) (end 93.345 78.74) (width 0.25) (layer F.Cu) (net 14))
 (segment (start 93.345 78.74) (end 95.885 76.2) (width 0.25) (layer F.Cu) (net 14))
 (segment (start 95.885 74.295) (end 95.885 76.2) (width 0.25) (layer F.Cu) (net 14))
 (segment (start 67.31 95.25) (end 59.69 95.25) (width 0.25) (layer F.Cu) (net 14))
 (segment (start 68.58 93.98) (end 67.31 95.25) (width 0.25) (layer F.Cu) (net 14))
 (segment (start 76.2 93.98) (end 68.58 93.98) (width 0.25) (layer F.Cu) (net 14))
 (segment (start 83.18359 74.295) (end 85.725 74.295) (width 0.25) (layer F.Cu) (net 1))
 (segment (start 80.00859 77.47) (end 83.18359 74.295) (width 0.25) (layer F.Cu) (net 1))
 (segment (start 69.85 77.47) (end 80.00859 77.47) (width 0.25) (layer F.Cu) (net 1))
 (segment (start 91.44 68.58) (end 104.14 68.58) (width 0.25) (layer F.Cu) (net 1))
 (segment (start 85.725 74.295) (end 91.44 68.58) (width 0.25) (layer F.Cu) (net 1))
 (segment (start 85.725 81.915) (end 85.725 86.995) (width 0.25) (layer F.Cu) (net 1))
 (segment (start 85.725 81.915) (end 85.725 74.295) (width 0.25) (layer B.Cu) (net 1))
 (segment (start 85.725 86.995) (end 85.725 94.615) (width 0.25) (layer B.Cu) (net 1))
 (segment (start 104.14 71.12) (end 104.14 87.63) (width 1.5) (layer F.Cu) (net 29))
 (segment (start 104.14 87.63) (end 101.6 90.17) (width 1.5) (layer F.Cu) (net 29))
 (segment (start 101.6 90.17) (end 97.79 90.17) (width 1.5) (layer F.Cu) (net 29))
 (segment (start 97.79 90.17) (end 95.885 92.075) (width 1.5) (layer F.Cu) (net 29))
 (segment (start 95.885 92.075) (end 89.535 92.075) (width 1.5) (layer F.Cu) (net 29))
 (segment (start 89.535 92.075) (end 88.265 93.345) (width 1.5) (layer F.Cu) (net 29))
 (segment (start 88.265 93.345) (end 88.265 94.615) (width 1.5) (layer F.Cu) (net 29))
 (segment (start 104.14 71.12) (end 104.14 74.295) (width 1.5) (layer B.Cu) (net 29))
 (segment (start 104.14 74.295) (end 101.6 76.835) (width 1.5) (layer B.Cu) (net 29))
 (segment (start 101.6 76.835) (end 91.44 76.835) (width 1.5) (layer B.Cu) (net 29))
 (segment (start 91.44 76.835) (end 88.265 80.01) (width 1.5) (layer B.Cu) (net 29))
 (segment (start 88.265 80.01) (end 88.265 81.915) (width 1.5) (layer B.Cu) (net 29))
 (segment (start 88.265 80.645) (end 88.265 81.915) (width 1) (layer B.Cu) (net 29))
 (segment (start 91.44 76.835) (end 88.265 80.645) (width 1) (layer B.Cu) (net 29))
 (segment (start 101.6 76.835) (end 91.44 76.835) (width 1) (layer B.Cu) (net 29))
 (segment (start 104.14 74.295) (end 101.6 76.835) (width 1) (layer B.Cu) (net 29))
 (segment (start 97.79 90.17) (end 95.885 92.075) (width 1) (layer F.Cu) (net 29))
 (segment (start 101.6 90.17) (end 97.79 90.17) (width 1) (layer F.Cu) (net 29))
 (segment (start 104.14 87.63) (end 101.6 90.17) (width 1) (layer F.Cu) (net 29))
 (segment (start 88.265 86.995) (end 86.995 85.725) (width 0.25) (layer B.Cu) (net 2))
 (segment (start 86.995 75.565) (end 88.265 74.295) (width 0.25) (layer B.Cu) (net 2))
 (segment (start 86.995 85.725) (end 86.995 75.565) (width 0.25) (layer B.Cu) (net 2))
 (segment (start 88.265 74.295) (end 86.36 76.2) (width 0.25) (layer F.Cu) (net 2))
 (segment (start 67.31 77.47) (end 59.69 77.47) (width 0.25) (layer F.Cu) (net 2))
 (segment (start 68.58 78.74) (end 67.31 77.47) (width 0.25) (layer F.Cu) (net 2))
 (segment (start 79.375 78.74) (end 68.58 78.74) (width 0.25) (layer F.Cu) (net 2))
 (segment (start 81.915 76.2) (end 79.375 78.74) (width 0.25) (layer F.Cu) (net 2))
 (segment (start 86.36 76.2) (end 81.915 76.2) (width 0.25) (layer F.Cu) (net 2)))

